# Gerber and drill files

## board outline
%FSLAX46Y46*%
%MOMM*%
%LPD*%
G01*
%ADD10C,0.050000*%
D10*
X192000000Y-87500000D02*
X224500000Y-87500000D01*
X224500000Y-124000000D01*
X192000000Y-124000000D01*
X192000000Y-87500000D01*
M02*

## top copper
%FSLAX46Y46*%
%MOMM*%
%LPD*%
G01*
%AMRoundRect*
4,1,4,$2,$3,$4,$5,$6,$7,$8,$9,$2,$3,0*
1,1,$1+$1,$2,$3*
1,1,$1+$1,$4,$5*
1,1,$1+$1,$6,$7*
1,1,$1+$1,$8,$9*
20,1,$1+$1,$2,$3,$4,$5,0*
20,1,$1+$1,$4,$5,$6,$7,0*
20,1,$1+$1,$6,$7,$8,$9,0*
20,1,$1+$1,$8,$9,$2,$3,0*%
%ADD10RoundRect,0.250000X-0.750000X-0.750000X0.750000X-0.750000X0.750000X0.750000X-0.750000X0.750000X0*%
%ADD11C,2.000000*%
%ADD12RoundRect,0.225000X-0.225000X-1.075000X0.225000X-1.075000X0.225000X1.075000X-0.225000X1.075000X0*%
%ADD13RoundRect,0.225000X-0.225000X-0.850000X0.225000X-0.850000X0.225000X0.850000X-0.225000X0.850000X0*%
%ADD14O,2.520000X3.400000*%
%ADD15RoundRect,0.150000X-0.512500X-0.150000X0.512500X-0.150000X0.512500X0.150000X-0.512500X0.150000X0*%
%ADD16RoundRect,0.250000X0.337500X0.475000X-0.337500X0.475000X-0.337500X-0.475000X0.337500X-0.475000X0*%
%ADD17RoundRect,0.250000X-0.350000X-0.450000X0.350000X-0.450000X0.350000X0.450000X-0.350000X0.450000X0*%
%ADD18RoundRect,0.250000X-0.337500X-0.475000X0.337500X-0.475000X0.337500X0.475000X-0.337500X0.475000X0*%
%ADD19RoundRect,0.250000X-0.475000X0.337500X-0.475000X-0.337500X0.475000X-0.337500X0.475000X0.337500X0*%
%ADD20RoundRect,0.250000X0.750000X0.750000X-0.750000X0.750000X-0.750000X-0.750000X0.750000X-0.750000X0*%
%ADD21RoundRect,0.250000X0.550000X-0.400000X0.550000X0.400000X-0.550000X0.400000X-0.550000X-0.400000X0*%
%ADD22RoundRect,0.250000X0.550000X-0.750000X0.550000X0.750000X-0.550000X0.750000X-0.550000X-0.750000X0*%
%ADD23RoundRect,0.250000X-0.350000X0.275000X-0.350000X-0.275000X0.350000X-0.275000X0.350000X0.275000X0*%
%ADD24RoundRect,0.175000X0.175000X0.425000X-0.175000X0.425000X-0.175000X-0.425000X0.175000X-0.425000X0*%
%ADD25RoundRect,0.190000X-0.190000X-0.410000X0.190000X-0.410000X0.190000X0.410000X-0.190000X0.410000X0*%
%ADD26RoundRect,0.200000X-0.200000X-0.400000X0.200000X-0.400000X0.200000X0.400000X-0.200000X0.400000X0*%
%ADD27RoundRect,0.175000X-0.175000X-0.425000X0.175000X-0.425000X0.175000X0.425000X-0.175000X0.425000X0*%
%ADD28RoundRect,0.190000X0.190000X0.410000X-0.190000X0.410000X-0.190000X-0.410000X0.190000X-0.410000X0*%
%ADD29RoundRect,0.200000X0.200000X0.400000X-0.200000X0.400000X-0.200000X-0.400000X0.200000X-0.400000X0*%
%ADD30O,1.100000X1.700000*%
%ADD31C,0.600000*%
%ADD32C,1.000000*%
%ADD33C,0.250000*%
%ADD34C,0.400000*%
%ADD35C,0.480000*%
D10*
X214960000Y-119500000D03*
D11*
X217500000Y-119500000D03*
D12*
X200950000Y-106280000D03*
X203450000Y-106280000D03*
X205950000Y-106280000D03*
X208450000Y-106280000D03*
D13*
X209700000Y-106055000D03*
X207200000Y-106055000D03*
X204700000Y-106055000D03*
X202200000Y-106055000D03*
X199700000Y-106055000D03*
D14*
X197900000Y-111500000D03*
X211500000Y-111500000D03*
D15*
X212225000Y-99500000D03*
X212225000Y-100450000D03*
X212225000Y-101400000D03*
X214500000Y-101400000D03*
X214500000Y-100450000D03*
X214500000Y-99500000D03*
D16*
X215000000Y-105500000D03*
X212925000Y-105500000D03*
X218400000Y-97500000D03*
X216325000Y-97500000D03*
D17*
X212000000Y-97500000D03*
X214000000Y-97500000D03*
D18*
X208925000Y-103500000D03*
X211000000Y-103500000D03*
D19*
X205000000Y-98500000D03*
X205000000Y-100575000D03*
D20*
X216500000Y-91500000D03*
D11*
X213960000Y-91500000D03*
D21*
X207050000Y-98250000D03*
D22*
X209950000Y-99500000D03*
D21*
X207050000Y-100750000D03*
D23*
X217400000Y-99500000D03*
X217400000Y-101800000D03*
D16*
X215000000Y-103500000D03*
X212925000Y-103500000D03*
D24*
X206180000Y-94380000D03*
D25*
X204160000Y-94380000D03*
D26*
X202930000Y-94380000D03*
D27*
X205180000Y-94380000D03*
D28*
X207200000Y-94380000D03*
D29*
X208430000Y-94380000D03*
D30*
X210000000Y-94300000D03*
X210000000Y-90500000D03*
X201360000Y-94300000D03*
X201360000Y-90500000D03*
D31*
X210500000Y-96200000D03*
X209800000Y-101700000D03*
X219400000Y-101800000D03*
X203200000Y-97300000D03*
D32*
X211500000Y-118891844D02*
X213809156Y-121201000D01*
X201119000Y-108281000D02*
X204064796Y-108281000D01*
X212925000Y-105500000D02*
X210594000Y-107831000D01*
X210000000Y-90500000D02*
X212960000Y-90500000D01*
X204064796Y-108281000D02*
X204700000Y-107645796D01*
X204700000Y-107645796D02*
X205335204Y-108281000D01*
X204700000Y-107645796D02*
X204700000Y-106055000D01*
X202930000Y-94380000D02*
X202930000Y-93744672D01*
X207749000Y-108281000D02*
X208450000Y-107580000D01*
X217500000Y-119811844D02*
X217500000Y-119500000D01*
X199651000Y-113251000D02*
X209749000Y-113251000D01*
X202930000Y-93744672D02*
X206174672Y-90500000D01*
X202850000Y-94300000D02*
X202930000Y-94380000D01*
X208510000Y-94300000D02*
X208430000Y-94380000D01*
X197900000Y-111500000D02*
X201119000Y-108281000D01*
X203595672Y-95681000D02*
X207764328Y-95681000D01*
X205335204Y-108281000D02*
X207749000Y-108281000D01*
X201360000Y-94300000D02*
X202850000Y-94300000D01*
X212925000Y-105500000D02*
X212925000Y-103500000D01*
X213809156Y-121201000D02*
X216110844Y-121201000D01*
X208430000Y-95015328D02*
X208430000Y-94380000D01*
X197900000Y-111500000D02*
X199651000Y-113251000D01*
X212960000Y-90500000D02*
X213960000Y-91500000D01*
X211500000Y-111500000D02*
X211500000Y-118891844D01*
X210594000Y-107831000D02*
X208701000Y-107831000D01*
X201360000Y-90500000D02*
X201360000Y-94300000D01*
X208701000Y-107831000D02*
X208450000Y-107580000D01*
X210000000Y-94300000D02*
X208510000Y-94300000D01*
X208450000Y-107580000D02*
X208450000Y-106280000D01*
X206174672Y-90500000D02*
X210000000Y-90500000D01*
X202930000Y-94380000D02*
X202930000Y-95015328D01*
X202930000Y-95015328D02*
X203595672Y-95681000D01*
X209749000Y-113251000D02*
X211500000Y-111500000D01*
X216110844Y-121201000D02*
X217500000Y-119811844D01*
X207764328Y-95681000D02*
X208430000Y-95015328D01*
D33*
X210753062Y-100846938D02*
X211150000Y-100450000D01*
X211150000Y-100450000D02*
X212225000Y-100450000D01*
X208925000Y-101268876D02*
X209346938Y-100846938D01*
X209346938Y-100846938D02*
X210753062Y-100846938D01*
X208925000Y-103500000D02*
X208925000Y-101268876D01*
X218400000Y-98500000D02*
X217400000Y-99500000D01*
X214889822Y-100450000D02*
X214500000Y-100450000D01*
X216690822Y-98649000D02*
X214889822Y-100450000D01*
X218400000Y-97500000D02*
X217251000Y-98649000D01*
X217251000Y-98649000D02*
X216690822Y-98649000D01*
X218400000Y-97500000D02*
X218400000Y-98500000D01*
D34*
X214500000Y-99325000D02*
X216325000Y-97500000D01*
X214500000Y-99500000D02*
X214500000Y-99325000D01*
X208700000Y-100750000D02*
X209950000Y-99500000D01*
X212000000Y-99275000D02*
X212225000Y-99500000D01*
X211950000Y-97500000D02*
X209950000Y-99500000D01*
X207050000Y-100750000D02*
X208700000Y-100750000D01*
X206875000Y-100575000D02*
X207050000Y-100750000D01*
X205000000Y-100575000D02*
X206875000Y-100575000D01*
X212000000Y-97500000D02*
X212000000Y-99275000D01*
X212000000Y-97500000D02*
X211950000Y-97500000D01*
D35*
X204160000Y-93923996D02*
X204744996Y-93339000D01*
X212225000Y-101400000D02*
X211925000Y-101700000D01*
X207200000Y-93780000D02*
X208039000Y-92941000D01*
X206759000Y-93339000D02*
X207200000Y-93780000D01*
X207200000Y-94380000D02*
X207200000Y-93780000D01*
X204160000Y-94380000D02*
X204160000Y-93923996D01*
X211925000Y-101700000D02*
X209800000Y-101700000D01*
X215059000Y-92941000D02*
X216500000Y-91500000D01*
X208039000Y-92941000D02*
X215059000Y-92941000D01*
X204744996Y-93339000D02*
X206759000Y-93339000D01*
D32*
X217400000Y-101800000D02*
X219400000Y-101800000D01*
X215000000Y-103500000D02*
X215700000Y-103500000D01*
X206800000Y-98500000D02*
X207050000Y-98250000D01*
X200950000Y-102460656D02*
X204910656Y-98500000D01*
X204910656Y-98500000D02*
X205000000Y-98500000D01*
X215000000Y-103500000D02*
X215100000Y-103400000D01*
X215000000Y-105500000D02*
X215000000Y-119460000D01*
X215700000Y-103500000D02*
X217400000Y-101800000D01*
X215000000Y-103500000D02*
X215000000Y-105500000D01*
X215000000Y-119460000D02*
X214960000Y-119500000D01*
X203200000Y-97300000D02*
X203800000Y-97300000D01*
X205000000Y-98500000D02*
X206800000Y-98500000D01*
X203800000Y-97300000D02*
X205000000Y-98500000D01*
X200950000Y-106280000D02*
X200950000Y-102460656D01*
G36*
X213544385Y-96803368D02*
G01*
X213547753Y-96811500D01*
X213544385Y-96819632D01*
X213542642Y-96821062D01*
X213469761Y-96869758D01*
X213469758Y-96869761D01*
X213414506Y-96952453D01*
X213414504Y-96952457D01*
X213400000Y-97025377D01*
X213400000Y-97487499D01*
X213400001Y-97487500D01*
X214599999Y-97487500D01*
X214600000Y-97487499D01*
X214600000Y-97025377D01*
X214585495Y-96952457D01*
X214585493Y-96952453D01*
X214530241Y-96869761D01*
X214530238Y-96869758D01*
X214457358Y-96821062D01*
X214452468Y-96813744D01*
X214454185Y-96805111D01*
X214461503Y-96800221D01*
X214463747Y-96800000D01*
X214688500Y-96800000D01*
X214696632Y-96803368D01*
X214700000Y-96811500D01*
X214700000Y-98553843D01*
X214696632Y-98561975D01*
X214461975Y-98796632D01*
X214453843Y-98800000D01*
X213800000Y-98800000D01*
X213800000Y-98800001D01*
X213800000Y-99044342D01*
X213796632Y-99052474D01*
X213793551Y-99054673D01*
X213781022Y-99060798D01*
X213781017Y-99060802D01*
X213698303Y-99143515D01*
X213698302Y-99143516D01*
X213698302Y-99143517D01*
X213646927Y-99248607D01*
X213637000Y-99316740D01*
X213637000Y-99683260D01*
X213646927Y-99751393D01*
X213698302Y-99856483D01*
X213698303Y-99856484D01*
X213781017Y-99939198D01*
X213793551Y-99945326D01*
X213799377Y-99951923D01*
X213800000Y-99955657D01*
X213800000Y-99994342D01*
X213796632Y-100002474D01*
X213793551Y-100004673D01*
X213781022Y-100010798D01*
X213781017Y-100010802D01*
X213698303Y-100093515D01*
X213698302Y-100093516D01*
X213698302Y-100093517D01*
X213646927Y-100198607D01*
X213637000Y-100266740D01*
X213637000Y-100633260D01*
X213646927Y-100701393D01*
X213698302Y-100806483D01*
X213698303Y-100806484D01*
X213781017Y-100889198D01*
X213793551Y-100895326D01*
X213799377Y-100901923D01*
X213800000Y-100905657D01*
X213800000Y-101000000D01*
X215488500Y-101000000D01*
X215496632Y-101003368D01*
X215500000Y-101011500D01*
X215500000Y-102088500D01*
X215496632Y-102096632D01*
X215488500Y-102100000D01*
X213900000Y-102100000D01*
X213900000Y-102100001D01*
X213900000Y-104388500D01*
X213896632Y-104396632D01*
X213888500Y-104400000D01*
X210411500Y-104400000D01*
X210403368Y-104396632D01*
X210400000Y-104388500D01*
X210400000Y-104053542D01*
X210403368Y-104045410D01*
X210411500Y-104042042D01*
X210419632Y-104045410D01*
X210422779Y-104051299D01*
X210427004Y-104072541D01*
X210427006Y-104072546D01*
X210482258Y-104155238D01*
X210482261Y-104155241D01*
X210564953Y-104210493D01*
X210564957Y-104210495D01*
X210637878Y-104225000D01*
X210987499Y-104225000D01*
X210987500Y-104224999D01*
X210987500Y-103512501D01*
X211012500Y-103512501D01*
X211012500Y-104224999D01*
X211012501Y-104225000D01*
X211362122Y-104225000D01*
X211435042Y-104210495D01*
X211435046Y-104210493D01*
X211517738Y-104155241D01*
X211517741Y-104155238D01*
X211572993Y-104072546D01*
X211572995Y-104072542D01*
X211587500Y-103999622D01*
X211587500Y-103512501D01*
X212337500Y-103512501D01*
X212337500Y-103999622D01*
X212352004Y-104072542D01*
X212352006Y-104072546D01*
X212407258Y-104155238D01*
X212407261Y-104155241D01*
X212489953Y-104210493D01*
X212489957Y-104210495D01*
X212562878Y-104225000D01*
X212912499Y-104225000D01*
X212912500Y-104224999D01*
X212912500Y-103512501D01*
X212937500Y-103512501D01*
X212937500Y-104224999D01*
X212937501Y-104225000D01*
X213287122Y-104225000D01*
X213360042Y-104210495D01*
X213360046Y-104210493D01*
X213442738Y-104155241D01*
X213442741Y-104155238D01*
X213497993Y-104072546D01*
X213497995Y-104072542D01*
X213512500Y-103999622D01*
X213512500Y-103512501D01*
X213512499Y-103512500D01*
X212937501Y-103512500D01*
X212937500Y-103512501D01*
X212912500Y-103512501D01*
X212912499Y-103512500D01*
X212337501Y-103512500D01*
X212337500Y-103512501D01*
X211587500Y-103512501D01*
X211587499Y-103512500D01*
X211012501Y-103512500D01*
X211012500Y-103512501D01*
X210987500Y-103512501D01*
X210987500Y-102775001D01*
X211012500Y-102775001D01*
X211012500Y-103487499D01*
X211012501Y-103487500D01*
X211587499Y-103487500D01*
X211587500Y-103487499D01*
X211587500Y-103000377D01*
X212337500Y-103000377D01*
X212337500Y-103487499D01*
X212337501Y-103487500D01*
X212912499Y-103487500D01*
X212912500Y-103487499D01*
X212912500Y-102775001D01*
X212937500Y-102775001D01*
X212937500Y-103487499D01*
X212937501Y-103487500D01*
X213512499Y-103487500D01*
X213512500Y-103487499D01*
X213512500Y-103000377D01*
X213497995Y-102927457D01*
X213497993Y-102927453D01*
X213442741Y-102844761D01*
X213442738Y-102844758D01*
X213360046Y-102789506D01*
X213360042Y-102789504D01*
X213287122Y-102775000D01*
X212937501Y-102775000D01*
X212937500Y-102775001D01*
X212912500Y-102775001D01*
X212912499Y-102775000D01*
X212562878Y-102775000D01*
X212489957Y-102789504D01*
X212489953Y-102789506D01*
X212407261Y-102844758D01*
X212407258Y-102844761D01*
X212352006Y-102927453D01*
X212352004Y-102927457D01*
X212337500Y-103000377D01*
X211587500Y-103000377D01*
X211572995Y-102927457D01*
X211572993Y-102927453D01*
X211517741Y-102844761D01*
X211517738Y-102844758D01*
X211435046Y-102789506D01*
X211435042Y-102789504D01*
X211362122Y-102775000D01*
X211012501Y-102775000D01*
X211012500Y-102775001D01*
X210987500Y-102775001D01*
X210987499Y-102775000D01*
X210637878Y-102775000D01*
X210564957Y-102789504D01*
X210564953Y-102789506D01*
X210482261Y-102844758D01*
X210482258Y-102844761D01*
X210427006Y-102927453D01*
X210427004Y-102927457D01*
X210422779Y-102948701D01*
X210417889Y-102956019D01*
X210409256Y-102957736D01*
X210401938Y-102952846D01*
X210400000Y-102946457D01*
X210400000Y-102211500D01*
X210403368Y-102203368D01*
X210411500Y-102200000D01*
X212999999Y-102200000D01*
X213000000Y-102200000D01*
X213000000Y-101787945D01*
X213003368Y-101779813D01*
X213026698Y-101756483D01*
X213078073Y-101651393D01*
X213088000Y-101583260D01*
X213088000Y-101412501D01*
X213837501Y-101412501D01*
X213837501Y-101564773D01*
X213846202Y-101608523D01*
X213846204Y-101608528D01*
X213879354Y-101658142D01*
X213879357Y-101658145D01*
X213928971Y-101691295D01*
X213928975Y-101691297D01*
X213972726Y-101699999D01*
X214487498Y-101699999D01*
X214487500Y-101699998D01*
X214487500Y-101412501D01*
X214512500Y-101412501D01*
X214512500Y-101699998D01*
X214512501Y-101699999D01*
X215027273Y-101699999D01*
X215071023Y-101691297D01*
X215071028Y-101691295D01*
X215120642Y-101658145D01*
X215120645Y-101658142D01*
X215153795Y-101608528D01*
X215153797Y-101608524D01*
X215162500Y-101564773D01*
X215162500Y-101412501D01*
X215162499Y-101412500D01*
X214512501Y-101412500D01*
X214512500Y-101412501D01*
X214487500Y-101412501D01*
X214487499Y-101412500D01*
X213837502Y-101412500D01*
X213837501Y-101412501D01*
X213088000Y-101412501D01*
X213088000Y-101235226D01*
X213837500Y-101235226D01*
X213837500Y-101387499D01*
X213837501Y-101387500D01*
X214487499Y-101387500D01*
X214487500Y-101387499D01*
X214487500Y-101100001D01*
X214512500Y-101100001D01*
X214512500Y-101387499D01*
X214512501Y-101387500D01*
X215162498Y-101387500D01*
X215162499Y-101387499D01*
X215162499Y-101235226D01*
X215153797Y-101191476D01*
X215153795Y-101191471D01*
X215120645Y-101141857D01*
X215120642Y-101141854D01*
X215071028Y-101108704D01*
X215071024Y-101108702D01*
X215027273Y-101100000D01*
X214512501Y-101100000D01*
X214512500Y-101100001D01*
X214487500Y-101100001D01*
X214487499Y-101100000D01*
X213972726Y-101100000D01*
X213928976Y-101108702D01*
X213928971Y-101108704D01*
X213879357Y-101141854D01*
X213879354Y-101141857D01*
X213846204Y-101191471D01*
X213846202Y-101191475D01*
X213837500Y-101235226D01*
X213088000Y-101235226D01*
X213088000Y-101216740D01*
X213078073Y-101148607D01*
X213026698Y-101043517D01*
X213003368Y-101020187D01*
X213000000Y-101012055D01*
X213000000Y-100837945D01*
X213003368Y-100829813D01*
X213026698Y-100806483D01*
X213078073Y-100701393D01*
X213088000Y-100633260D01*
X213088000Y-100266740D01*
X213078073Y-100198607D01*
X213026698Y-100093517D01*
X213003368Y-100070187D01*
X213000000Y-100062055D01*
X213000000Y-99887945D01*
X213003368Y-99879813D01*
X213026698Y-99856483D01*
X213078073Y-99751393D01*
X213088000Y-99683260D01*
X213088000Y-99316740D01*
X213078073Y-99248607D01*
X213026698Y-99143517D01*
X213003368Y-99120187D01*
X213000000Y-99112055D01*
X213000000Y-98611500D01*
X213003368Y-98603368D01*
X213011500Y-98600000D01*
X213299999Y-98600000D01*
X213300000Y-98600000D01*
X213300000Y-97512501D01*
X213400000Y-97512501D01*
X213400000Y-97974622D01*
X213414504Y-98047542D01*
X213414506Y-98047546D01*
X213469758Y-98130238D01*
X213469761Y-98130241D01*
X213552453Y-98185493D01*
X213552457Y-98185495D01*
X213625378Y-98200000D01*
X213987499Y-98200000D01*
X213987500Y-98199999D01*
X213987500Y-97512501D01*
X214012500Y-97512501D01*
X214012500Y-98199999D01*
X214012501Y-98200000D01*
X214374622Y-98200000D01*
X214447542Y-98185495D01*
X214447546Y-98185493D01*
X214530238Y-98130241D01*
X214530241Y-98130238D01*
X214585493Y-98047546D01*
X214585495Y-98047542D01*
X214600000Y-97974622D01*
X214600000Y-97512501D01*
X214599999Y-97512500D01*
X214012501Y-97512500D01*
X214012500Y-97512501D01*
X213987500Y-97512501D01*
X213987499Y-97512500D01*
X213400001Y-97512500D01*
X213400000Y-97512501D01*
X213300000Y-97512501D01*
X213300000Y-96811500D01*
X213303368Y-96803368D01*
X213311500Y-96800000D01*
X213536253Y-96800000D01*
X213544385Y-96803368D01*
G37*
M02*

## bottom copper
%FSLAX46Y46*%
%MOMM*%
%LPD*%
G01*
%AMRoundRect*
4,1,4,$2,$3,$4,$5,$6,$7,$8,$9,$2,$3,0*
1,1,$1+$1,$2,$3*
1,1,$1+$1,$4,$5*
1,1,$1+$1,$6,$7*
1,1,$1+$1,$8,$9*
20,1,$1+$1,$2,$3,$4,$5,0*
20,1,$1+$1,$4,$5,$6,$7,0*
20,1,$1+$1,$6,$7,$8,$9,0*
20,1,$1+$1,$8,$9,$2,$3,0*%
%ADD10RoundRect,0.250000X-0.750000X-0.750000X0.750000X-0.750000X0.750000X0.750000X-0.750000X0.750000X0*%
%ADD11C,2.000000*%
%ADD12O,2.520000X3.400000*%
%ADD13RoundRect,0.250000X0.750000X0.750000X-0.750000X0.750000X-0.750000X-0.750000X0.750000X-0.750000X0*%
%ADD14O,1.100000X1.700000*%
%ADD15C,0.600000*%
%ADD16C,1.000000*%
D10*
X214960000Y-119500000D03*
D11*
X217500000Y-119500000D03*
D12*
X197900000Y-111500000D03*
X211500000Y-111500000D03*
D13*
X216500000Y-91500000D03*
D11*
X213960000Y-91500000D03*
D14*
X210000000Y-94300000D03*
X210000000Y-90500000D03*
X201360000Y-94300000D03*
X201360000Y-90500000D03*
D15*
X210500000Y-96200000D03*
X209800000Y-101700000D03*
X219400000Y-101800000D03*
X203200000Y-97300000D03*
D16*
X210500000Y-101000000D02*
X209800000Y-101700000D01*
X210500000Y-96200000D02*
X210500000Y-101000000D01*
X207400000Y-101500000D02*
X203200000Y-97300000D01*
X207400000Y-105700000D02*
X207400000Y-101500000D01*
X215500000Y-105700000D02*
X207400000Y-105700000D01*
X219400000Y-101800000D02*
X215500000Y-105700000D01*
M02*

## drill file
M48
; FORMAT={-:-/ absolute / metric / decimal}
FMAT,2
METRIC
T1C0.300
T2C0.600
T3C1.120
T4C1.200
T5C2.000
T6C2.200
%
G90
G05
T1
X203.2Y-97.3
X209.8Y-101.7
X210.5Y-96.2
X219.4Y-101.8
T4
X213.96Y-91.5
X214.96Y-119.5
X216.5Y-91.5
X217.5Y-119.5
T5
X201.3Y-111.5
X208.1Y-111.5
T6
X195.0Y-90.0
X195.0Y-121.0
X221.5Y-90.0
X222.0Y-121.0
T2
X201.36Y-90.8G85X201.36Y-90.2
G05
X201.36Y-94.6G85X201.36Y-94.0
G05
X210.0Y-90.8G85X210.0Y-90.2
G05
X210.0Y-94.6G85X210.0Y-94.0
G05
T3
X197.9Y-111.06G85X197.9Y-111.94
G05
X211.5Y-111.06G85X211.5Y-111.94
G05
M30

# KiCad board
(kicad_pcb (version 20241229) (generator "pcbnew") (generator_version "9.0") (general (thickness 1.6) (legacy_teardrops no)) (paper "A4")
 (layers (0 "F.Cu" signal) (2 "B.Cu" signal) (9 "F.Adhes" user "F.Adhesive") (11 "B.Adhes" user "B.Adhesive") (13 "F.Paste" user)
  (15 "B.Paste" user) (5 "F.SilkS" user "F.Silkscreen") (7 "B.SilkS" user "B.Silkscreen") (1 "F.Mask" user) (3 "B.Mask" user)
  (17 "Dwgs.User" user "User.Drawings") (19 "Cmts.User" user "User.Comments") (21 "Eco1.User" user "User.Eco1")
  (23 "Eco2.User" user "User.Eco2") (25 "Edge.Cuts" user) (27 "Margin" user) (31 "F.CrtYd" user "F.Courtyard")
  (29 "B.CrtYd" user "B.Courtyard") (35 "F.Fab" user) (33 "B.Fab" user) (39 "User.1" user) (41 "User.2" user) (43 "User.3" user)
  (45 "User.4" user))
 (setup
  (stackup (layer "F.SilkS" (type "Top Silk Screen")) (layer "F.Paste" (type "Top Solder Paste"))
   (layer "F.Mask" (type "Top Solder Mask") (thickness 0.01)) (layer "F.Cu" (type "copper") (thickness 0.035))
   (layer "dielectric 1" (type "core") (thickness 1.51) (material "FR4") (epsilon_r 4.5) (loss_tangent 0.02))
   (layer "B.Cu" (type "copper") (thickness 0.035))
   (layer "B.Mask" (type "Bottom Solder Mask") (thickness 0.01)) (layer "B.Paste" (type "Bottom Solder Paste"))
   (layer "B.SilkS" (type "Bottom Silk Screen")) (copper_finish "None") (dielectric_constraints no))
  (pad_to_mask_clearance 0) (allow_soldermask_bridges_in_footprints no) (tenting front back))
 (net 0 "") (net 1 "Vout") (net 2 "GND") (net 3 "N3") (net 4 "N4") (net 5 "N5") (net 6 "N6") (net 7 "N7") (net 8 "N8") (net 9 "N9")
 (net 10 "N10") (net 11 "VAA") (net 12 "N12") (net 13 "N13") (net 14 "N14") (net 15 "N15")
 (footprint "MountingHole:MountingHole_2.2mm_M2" (layer "F.Cu") (at 195 121)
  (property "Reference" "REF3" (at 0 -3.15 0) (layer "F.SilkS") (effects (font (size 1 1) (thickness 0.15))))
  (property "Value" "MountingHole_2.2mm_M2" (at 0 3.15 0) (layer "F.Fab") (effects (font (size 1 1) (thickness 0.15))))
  (pad "" np_thru_hole circle (at 0 0) (size 2.2 2.2) (drill 2.2) (layers "*.Cu" "*.Mask")))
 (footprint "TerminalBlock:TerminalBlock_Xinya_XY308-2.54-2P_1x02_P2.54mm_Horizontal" (layer "F.Cu") (at 214.96 119.5)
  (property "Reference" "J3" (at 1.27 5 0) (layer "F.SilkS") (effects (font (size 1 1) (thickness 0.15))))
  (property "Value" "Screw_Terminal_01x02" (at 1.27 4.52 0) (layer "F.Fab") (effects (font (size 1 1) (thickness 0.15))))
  (pad "1" thru_hole roundrect (at 0 0) (size 2 2) (drill 1.2) (layers "*.Cu" "*.Mask") (remove_unused_layers no) (roundrect_rratio 0.125)
   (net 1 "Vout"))
  (pad "2" thru_hole circle (at 2.54 0) (size 2 2) (drill 1.2) (layers "*.Cu" "*.Mask") (remove_unused_layers no) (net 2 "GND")))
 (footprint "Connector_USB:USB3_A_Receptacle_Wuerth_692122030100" (layer "F.Cu") (at 204.7 114.95)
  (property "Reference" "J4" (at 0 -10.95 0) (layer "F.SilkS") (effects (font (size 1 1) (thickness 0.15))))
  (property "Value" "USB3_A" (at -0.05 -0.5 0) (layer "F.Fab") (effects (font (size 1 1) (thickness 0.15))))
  (pad "" np_thru_hole circle (at -3.4 -3.45) (size 2 2) (drill 2) (layers "*.Cu" "*.Mask"))
  (pad "" np_thru_hole circle (at 3.4 -3.45) (size 2 2) (drill 2) (layers "*.Cu" "*.Mask"))
  (pad "1" smd roundrect (at -3.75 -8.67) (size 0.9 2.6) (layers "F.Cu" "F.Mask" "F.Paste") (roundrect_rratio 0.25) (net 1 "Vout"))
  (pad "2" smd roundrect (at -1.25 -8.67) (size 0.9 2.6) (layers "F.Cu" "F.Mask" "F.Paste") (roundrect_rratio 0.25) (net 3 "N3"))
  (pad "3" smd roundrect (at 1.25 -8.67) (size 0.9 2.6) (layers "F.Cu" "F.Mask" "F.Paste") (roundrect_rratio 0.25) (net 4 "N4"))
  (pad "4" smd roundrect (at 3.75 -8.67) (size 0.9 2.6) (layers "F.Cu" "F.Mask" "F.Paste") (roundrect_rratio 0.25) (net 2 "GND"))
  (pad "5" smd roundrect (at 5 -8.895) (size 0.9 2.15) (layers "F.Cu" "F.Mask" "F.Paste") (roundrect_rratio 0.25) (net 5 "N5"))
  (pad "6" smd roundrect (at 2.5 -8.895) (size 0.9 2.15) (layers "F.Cu" "F.Mask" "F.Paste") (roundrect_rratio 0.25) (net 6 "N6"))
  (pad "7" smd roundrect (at 0 -8.895) (size 0.9 2.15) (layers "F.Cu" "F.Mask" "F.Paste") (roundrect_rratio 0.25) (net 2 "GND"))
  (pad "8" smd roundrect (at -2.5 -8.895) (size 0.9 2.15) (layers "F.Cu" "F.Mask" "F.Paste") (roundrect_rratio 0.25) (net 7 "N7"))
  (pad "9" smd roundrect (at -5 -8.895) (size 0.9 2.15) (layers "F.Cu" "F.Mask" "F.Paste") (roundrect_rratio 0.25) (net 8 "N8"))
  (pad "10" thru_hole oval (at -6.8 -3.45) (size 2.52 3.4) (drill oval 1.12 2) (layers "*.Cu" "*.Mask") (remove_unused_layers no)
   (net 2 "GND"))
  (pad "10" thru_hole oval (at 6.8 -3.45) (size 2.52 3.4) (drill oval 1.12 2) (layers "*.Cu" "*.Mask") (remove_unused_layers no)
   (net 2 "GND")))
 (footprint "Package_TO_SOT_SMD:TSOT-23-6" (layer "F.Cu") (at 213.3625 100.45)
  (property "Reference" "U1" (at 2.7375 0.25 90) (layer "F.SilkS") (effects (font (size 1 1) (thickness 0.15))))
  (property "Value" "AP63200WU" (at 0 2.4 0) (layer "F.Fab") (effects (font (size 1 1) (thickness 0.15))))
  (pad "1" smd roundrect (at -1.1375 -0.95) (size 1.325 0.6) (layers "F.Cu" "F.Mask" "F.Paste") (roundrect_rratio 0.25) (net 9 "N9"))
  (pad "2" smd roundrect (at -1.1375 0) (size 1.325 0.6) (layers "F.Cu" "F.Mask" "F.Paste") (roundrect_rratio 0.25) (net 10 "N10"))
  (pad "3" smd roundrect (at -1.1375 0.95) (size 1.325 0.6) (layers "F.Cu" "F.Mask" "F.Paste") (roundrect_rratio 0.25) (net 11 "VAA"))
  (pad "4" smd roundrect (at 1.1375 0.95) (size 1.325 0.6) (layers "F.Cu" "F.Mask" "F.Paste") (roundrect_rratio 0.25) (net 2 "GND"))
  (pad "5" smd roundrect (at 1.1375 0) (size 1.325 0.6) (layers "F.Cu" "F.Mask" "F.Paste") (roundrect_rratio 0.25) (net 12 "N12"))
  (pad "6" smd roundrect (at 1.1375 -0.95) (size 1.325 0.6) (layers "F.Cu" "F.Mask" "F.Paste") (roundrect_rratio 0.25) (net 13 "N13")))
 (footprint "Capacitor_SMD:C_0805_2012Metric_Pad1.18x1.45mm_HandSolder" (layer "F.Cu") (at 213.9625 105.5 180)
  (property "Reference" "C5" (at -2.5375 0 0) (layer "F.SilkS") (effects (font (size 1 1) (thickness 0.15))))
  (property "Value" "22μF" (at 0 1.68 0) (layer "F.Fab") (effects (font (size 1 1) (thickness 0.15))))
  (pad "1" smd roundrect (at -1.0375 0 180) (size 1.175 1.45) (layers "F.Cu" "F.Mask" "F.Paste") (roundrect_rratio 0.212766) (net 1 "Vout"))
  (pad "2" smd roundrect (at 1.0375 0 180) (size 1.175 1.45) (layers "F.Cu" "F.Mask" "F.Paste") (roundrect_rratio 0.212766) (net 2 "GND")))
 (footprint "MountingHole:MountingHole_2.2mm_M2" (layer "F.Cu") (at 222 121)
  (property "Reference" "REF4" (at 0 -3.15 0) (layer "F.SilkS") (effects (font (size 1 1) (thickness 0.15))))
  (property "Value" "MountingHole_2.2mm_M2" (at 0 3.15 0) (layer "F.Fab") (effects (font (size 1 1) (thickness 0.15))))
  (pad "" np_thru_hole circle (at 0 0) (size 2.2 2.2) (drill 2.2) (layers "*.Cu" "*.Mask")))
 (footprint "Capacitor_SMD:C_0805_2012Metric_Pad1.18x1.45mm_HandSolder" (layer "F.Cu") (at 217.3625 97.5 180)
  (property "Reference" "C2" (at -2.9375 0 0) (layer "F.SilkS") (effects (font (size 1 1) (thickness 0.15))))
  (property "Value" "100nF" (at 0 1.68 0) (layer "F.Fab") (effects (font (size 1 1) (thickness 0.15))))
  (pad "1" smd roundrect (at -1.0375 0 180) (size 1.175 1.45) (layers "F.Cu" "F.Mask" "F.Paste") (roundrect_rratio 0.212766) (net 12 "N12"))
  (pad "2" smd roundrect (at 1.0375 0 180) (size 1.175 1.45) (layers "F.Cu" "F.Mask" "F.Paste") (roundrect_rratio 0.212766) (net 13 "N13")))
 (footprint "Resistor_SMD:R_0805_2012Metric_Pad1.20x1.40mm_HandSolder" (layer "F.Cu") (at 213 97.5)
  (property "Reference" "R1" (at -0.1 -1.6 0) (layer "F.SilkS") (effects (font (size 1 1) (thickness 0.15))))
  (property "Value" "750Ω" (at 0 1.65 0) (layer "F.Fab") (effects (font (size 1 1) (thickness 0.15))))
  (pad "1" smd roundrect (at -1 0) (size 1.2 1.4) (layers "F.Cu" "F.Mask" "F.Paste") (roundrect_rratio 0.208333) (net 9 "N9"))
  (pad "2" smd roundrect (at 1 0) (size 1.2 1.4) (layers "F.Cu" "F.Mask" "F.Paste") (roundrect_rratio 0.208333) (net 2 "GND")))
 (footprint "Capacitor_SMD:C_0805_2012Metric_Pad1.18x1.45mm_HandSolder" (layer "F.Cu") (at 209.9625 103.5)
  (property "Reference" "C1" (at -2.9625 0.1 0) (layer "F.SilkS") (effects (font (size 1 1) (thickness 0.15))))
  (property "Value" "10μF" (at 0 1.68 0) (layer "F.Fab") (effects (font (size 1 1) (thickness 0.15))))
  (pad "1" smd roundrect (at -1.0375 0) (size 1.175 1.45) (layers "F.Cu" "F.Mask" "F.Paste") (roundrect_rratio 0.212766) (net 10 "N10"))
  (pad "2" smd roundrect (at 1.0375 0) (size 1.175 1.45) (layers "F.Cu" "F.Mask" "F.Paste") (roundrect_rratio 0.212766) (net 2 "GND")))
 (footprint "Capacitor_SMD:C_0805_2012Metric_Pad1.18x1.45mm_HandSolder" (layer "F.Cu") (at 205 99.5375 -90)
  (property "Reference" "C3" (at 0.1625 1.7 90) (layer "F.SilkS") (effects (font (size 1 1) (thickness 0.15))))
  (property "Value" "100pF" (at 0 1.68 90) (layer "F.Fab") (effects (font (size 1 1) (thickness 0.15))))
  (pad "1" smd roundrect (at -1.0375 0 270) (size 1.175 1.45) (layers "F.Cu" "F.Mask" "F.Paste") (roundrect_rratio 0.212766) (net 1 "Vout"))
  (pad "2" smd roundrect (at 1.0375 0 270) (size 1.175 1.45) (layers "F.Cu" "F.Mask" "F.Paste") (roundrect_rratio 0.212766) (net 9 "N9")))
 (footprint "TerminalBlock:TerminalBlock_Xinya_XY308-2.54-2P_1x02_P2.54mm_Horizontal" (layer "F.Cu") (at 216.5 91.5 180)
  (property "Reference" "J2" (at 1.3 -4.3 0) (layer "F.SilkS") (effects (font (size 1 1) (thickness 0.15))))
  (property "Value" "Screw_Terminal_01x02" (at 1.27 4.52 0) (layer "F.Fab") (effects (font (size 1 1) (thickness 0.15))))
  (pad "1" thru_hole roundrect (at 0 0 180) (size 2 2) (drill 1.2) (layers "*.Cu" "*.Mask") (remove_unused_layers no)
   (roundrect_rratio 0.125) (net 11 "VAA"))
  (pad "2" thru_hole circle (at 2.54 0 180) (size 2 2) (drill 1.2) (layers "*.Cu" "*.Mask") (remove_unused_layers no) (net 2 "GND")))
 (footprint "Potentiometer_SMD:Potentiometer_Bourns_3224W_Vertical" (layer "F.Cu") (at 208.5 99.5 90)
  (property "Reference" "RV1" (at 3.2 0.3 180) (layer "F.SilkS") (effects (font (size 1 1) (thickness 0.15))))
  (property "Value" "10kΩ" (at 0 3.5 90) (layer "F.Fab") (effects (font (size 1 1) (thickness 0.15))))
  (pad "1" smd roundrect (at 1.25 -1.45 90) (size 1.3 1.6) (layers "F.Cu" "F.Mask" "F.Paste") (roundrect_rratio 0.192308) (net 1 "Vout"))
  (pad "2" smd roundrect (at 0 1.45 90) (size 2 1.6) (layers "F.Cu" "F.Mask" "F.Paste") (roundrect_rratio 0.15625) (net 9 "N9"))
  (pad "3" smd roundrect (at -1.25 -1.45 90) (size 1.3 1.6) (layers "F.Cu" "F.Mask" "F.Paste") (roundrect_rratio 0.192308) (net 9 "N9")))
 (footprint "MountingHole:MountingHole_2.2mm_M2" (layer "F.Cu") (at 221.5 90)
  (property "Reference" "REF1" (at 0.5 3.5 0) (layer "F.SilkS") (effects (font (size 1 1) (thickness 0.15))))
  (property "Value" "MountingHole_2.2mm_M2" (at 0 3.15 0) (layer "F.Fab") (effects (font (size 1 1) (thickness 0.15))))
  (pad "" np_thru_hole circle (at 0 0) (size 2.2 2.2) (drill 2.2) (layers "*.Cu" "*.Mask")))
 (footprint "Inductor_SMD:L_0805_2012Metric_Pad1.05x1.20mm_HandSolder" (layer "F.Cu") (at 217.4 100.65 -90)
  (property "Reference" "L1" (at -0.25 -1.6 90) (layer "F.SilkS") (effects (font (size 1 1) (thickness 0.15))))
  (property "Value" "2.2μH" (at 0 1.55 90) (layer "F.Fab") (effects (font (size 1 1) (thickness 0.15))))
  (pad "1" smd roundrect (at -1.15 0 270) (size 1.05 1.2) (layers "F.Cu" "F.Mask" "F.Paste") (roundrect_rratio 0.238095) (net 12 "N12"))
  (pad "2" smd roundrect (at 1.15 0 270) (size 1.05 1.2) (layers "F.Cu" "F.Mask" "F.Paste") (roundrect_rratio 0.238095) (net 1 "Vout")))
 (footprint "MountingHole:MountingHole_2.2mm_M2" (layer "F.Cu") (at 195 90)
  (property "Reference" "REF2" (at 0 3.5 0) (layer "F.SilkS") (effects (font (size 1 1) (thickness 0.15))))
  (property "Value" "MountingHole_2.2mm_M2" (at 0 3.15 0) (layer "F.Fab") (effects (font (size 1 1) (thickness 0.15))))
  (pad "" np_thru_hole circle (at 0 0) (size 2.2 2.2) (drill 2.2) (layers "*.Cu" "*.Mask")))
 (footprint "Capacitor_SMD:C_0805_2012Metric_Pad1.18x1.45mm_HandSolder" (layer "F.Cu") (at 213.9625 103.5 180)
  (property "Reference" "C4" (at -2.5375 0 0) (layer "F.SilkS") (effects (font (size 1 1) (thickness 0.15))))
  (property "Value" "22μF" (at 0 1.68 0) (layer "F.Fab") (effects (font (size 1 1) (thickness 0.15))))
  (pad "1" smd roundrect (at -1.0375 0 180) (size 1.175 1.45) (layers "F.Cu" "F.Mask" "F.Paste") (roundrect_rratio 0.212766) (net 1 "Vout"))
  (pad "2" smd roundrect (at 1.0375 0 180) (size 1.175 1.45) (layers "F.Cu" "F.Mask" "F.Paste") (roundrect_rratio 0.212766) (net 2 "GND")))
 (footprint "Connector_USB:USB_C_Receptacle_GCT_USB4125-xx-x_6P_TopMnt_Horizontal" (layer "F.Cu") (at 205.68 91.3 180)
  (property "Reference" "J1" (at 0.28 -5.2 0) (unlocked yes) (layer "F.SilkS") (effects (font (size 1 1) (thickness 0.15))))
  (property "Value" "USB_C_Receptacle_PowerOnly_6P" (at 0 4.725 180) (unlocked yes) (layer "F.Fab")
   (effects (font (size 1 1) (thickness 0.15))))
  (pad "A5" smd roundrect (at -0.5 -3.08 180) (size 0.7 1.2) (layers "F.Cu" "F.Mask" "F.Paste") (roundrect_rratio 0.25) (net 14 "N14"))
  (pad "A9" smd roundrect (at 1.52 -3.08) (size 0.76 1.2) (layers "F.Cu" "F.Mask" "F.Paste") (roundrect_rratio 0.25) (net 11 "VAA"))
  (pad "A12" smd roundrect (at 2.75 -3.08) (size 0.8 1.2) (layers "F.Cu" "F.Mask" "F.Paste") (roundrect_rratio 0.25) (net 2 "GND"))
  (pad "B5" smd roundrect (at 0.5 -3.08) (size 0.7 1.2) (layers "F.Cu" "F.Mask" "F.Paste") (roundrect_rratio 0.25) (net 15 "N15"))
  (pad "B9" smd roundrect (at -1.52 -3.08 180) (size 0.76 1.2) (layers "F.Cu" "F.Mask" "F.Paste") (roundrect_rratio 0.25) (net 11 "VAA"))
  (pad "B12" smd roundrect (at -2.75 -3.08 180) (size 0.8 1.2) (layers "F.Cu" "F.Mask" "F.Paste") (roundrect_rratio 0.25) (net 2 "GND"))
  (pad "S1" thru_hole oval (at -4.32 -3 180) (size 1.1 1.7) (drill oval 0.6 1.2) (layers "*.Cu" "*.Mask" "F.Paste")
   (remove_unused_layers no) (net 2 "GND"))
  (pad "S1" thru_hole oval (at -4.32 0.8 180) (size 1.1 1.7) (drill oval 0.6 1.2) (layers "*.Cu" "*.Mask" "F.Paste")
   (remove_unused_layers no) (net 2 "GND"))
  (pad "S1" thru_hole oval (at 4.32 -3 180) (size 1.1 1.7) (drill oval 0.6 1.2) (layers "*.Cu" "*.Mask" "F.Paste") (remove_unused_layers no)
   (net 2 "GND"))
  (pad "S1" thru_hole oval (at 4.32 0.8 180) (size 1.1 1.7) (drill oval 0.6 1.2) (layers "*.Cu" "*.Mask" "F.Paste")
   (remove_unused_layers no) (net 2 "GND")))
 (gr_rect (start 192 87.5) (end 224.5 124) (stroke (width 0.05) (type default)) (fill no) (layer "Edge.Cuts"))
 (segment (start 211.5 118.891844) (end 213.809156 121.201) (width 1) (layer "F.Cu") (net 2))
 (segment (start 201.119 108.281) (end 204.064796 108.281) (width 1) (layer "F.Cu") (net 2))
 (segment (start 212.925 105.5) (end 210.594 107.831) (width 1) (layer "F.Cu") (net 2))
 (segment (start 210 90.5) (end 212.96 90.5) (width 1) (layer "F.Cu") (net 2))
 (segment (start 204.064796 108.281) (end 204.7 107.645796) (width 1) (layer "F.Cu") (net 2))
 (segment (start 204.7 107.645796) (end 205.335204 108.281) (width 1) (layer "F.Cu") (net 2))
 (segment (start 204.7 107.645796) (end 204.7 106.055) (width 1) (layer "F.Cu") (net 2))
 (segment (start 202.93 94.38) (end 202.93 93.744672) (width 1) (layer "F.Cu") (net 2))
 (segment (start 207.749 108.281) (end 208.45 107.58) (width 1) (layer "F.Cu") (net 2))
 (segment (start 217.5 119.811844) (end 217.5 119.5) (width 1) (layer "F.Cu") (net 2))
 (segment (start 199.651 113.251) (end 209.749 113.251) (width 1) (layer "F.Cu") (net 2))
 (segment (start 202.93 93.744672) (end 206.174672 90.5) (width 1) (layer "F.Cu") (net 2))
 (segment (start 202.85 94.3) (end 202.93 94.38) (width 1) (layer "F.Cu") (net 2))
 (segment (start 208.51 94.3) (end 208.43 94.38) (width 1) (layer "F.Cu") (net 2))
 (segment (start 197.9 111.5) (end 201.119 108.281) (width 1) (layer "F.Cu") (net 2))
 (segment (start 203.595672 95.681) (end 207.764328 95.681) (width 1) (layer "F.Cu") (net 2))
 (segment (start 205.335204 108.281) (end 207.749 108.281) (width 1) (layer "F.Cu") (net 2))
 (segment (start 201.36 94.3) (end 202.85 94.3) (width 1) (layer "F.Cu") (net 2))
 (segment (start 212.925 105.5) (end 212.925 103.5) (width 1) (layer "F.Cu") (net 2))
 (segment (start 213.809156 121.201) (end 216.110844 121.201) (width 1) (layer "F.Cu") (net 2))
 (segment (start 208.43 95.015328) (end 208.43 94.38) (width 1) (layer "F.Cu") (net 2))
 (segment (start 197.9 111.5) (end 199.651 113.251) (width 1) (layer "F.Cu") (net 2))
 (segment (start 212.96 90.5) (end 213.96 91.5) (width 1) (layer "F.Cu") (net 2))
 (segment (start 211.5 111.5) (end 211.5 118.891844) (width 1) (layer "F.Cu") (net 2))
 (segment (start 210.594 107.831) (end 208.701 107.831) (width 1) (layer "F.Cu") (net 2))
 (segment (start 201.36 90.5) (end 201.36 94.3) (width 1) (layer "F.Cu") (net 2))
 (segment (start 208.701 107.831) (end 208.45 107.58) (width 1) (layer "F.Cu") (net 2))
 (segment (start 210 94.3) (end 208.51 94.3) (width 1) (layer "F.Cu") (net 2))
 (segment (start 208.45 107.58) (end 208.45 106.28) (width 1) (layer "F.Cu") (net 2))
 (segment (start 206.174672 90.5) (end 210 90.5) (width 1) (layer "F.Cu") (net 2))
 (segment (start 202.93 94.38) (end 202.93 95.015328) (width 1) (layer "F.Cu") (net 2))
 (segment (start 202.93 95.015328) (end 203.595672 95.681) (width 1) (layer "F.Cu") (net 2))
 (segment (start 209.749 113.251) (end 211.5 111.5) (width 1) (layer "F.Cu") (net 2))
 (segment (start 216.110844 121.201) (end 217.5 119.811844) (width 1) (layer "F.Cu") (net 2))
 (segment (start 207.764328 95.681) (end 208.43 95.015328) (width 1) (layer "F.Cu") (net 2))
 (segment (start 210.753062 100.846938) (end 211.15 100.45) (width 0.25) (layer "F.Cu") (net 10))
 (segment (start 211.15 100.45) (end 212.225 100.45) (width 0.25) (layer "F.Cu") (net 10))
 (segment (start 208.925 101.268876) (end 209.346938 100.846938) (width 0.25) (layer "F.Cu") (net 10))
 (segment (start 209.346938 100.846938) (end 210.753062 100.846938) (width 0.25) (layer "F.Cu") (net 10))
 (segment (start 208.925 103.5) (end 208.925 101.268876) (width 0.25) (layer "F.Cu") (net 10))
 (segment (start 218.4 98.5) (end 217.4 99.5) (width 0.25) (layer "F.Cu") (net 12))
 (segment (start 214.889822 100.45) (end 214.5 100.45) (width 0.25) (layer "F.Cu") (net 12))
 (segment (start 216.690822 98.649) (end 214.889822 100.45) (width 0.25) (layer "F.Cu") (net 12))
 (segment (start 218.4 97.5) (end 217.251 98.649) (width 0.25) (layer "F.Cu") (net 12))
 (segment (start 217.251 98.649) (end 216.690822 98.649) (width 0.25) (layer "F.Cu") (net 12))
 (segment (start 218.4 97.5) (end 218.4 98.5) (width 0.25) (layer "F.Cu") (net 12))
 (segment (start 214.5 99.325) (end 216.325 97.5) (width 0.4) (layer "F.Cu") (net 13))
 (segment (start 214.5 99.5) (end 214.5 99.325) (width 0.4) (layer "F.Cu") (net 13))
 (segment (start 208.7 100.75) (end 209.95 99.5) (width 0.4) (layer "F.Cu") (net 9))
 (segment (start 212 99.275) (end 212.225 99.5) (width 0.4) (layer "F.Cu") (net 9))
 (segment (start 211.95 97.5) (end 209.95 99.5) (width 0.4) (layer "F.Cu") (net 9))
 (segment (start 207.05 100.75) (end 208.7 100.75) (width 0.4) (layer "F.Cu") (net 9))
 (segment (start 206.875 100.575) (end 207.05 100.75) (width 0.4) (layer "F.Cu") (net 9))
 (segment (start 205 100.575) (end 206.875 100.575) (width 0.4) (layer "F.Cu") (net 9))
 (segment (start 212 97.5) (end 212 99.275) (width 0.4) (layer "F.Cu") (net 9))
 (segment (start 212 97.5) (end 211.95 97.5) (width 0.4) (layer "F.Cu") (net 9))
 (segment (start 204.16 93.923996) (end 204.744996 93.339) (width 0.48) (layer "F.Cu") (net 11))
 (segment (start 212.225 101.4) (end 211.925 101.7) (width 0.48) (layer "F.Cu") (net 11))
 (segment (start 207.2 93.78) (end 208.039 92.941) (width 0.48) (layer "F.Cu") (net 11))
 (segment (start 206.759 93.339) (end 207.2 93.78) (width 0.48) (layer "F.Cu") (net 11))
 (segment (start 207.2 94.38) (end 207.2 93.78) (width 0.48) (layer "F.Cu") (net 11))
 (segment (start 204.16 94.38) (end 204.16 93.923996) (width 0.48) (layer "F.Cu") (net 11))
 (segment (start 211.925 101.7) (end 209.8 101.7) (width 0.48) (layer "F.Cu") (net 11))
 (segment (start 215.059 92.941) (end 216.5 91.5) (width 0.48) (layer "F.Cu") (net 11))
 (segment (start 208.039 92.941) (end 215.059 92.941) (width 0.48) (layer "F.Cu") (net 11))
 (segment (start 204.744996 93.339) (end 206.759 93.339) (width 0.48) (layer "F.Cu") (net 11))
 (via (at 210.5 96.2) (size 0.6) (drill 0.3) (layers "F.Cu" "B.Cu") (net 11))
 (via (at 209.8 101.7) (size 0.6) (drill 0.3) (layers "F.Cu" "B.Cu") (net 11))
 (segment (start 210.5 101) (end 209.8 101.7) (width 1) (layer "B.Cu") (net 11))
 (segment (start 210.5 96.2) (end 210.5 101) (width 1) (layer "B.Cu") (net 11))
 (segment (start 217.4 101.8) (end 219.4 101.8) (width 1) (layer "F.Cu") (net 1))
 (segment (start 215 103.5) (end 215.7 103.5) (width 1) (layer "F.Cu") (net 1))
 (segment (start 206.8 98.5) (end 207.05 98.25) (width 1) (layer "F.Cu") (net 1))
 (segment (start 200.95 102.460656) (end 204.910656 98.5) (width 1) (layer "F.Cu") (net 1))
 (segment (start 204.910656 98.5) (end 205 98.5) (width 1) (layer "F.Cu") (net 1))
 (segment (start 215 103.5) (end 215.1 103.4) (width 1) (layer "F.Cu") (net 1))
 (segment (start 215 105.5) (end 215 119.46) (width 1) (layer "F.Cu") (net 1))
 (segment (start 215.7 103.5) (end 217.4 101.8) (width 1) (layer "F.Cu") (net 1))
 (segment (start 215 103.5) (end 215 105.5) (width 1) (layer "F.Cu") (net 1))
 (segment (start 215 119.46) (end 214.96 119.5) (width 1) (layer "F.Cu") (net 1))
 (segment (start 203.2 97.3) (end 203.8 97.3) (width 1) (layer "F.Cu") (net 1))
 (segment (start 205 98.5) (end 206.8 98.5) (width 1) (layer "F.Cu") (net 1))
 (segment (start 203.8 97.3) (end 205 98.5) (width 1) (layer "F.Cu") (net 1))
 (segment (start 200.95 106.28) (end 200.95 102.460656) (width 1) (layer "F.Cu") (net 1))
 (via (at 219.4 101.8) (size 0.6) (drill 0.3) (layers "F.Cu" "B.Cu") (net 1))
 (via (at 203.2 97.3) (size 0.6) (drill 0.3) (layers "F.Cu" "B.Cu") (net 1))
 (segment (start 207.4 101.5) (end 203.2 97.3) (width 1) (layer "B.Cu") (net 1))
 (segment (start 207.4 105.7) (end 207.4 101.5) (width 1) (layer "B.Cu") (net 1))
 (segment (start 215.5 105.7) (end 207.4 105.7) (width 1) (layer "B.Cu") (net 1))
 (segment (start 219.4 101.8) (end 215.5 105.7) (width 1) (layer "B.Cu") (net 1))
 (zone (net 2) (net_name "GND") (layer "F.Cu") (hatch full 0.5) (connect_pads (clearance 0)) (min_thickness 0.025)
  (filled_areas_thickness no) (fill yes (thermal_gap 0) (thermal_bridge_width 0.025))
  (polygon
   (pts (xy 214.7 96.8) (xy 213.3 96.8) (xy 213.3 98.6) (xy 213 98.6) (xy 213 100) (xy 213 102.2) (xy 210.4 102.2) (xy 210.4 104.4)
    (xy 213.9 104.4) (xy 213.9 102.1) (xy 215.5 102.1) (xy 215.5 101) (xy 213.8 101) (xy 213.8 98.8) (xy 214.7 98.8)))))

